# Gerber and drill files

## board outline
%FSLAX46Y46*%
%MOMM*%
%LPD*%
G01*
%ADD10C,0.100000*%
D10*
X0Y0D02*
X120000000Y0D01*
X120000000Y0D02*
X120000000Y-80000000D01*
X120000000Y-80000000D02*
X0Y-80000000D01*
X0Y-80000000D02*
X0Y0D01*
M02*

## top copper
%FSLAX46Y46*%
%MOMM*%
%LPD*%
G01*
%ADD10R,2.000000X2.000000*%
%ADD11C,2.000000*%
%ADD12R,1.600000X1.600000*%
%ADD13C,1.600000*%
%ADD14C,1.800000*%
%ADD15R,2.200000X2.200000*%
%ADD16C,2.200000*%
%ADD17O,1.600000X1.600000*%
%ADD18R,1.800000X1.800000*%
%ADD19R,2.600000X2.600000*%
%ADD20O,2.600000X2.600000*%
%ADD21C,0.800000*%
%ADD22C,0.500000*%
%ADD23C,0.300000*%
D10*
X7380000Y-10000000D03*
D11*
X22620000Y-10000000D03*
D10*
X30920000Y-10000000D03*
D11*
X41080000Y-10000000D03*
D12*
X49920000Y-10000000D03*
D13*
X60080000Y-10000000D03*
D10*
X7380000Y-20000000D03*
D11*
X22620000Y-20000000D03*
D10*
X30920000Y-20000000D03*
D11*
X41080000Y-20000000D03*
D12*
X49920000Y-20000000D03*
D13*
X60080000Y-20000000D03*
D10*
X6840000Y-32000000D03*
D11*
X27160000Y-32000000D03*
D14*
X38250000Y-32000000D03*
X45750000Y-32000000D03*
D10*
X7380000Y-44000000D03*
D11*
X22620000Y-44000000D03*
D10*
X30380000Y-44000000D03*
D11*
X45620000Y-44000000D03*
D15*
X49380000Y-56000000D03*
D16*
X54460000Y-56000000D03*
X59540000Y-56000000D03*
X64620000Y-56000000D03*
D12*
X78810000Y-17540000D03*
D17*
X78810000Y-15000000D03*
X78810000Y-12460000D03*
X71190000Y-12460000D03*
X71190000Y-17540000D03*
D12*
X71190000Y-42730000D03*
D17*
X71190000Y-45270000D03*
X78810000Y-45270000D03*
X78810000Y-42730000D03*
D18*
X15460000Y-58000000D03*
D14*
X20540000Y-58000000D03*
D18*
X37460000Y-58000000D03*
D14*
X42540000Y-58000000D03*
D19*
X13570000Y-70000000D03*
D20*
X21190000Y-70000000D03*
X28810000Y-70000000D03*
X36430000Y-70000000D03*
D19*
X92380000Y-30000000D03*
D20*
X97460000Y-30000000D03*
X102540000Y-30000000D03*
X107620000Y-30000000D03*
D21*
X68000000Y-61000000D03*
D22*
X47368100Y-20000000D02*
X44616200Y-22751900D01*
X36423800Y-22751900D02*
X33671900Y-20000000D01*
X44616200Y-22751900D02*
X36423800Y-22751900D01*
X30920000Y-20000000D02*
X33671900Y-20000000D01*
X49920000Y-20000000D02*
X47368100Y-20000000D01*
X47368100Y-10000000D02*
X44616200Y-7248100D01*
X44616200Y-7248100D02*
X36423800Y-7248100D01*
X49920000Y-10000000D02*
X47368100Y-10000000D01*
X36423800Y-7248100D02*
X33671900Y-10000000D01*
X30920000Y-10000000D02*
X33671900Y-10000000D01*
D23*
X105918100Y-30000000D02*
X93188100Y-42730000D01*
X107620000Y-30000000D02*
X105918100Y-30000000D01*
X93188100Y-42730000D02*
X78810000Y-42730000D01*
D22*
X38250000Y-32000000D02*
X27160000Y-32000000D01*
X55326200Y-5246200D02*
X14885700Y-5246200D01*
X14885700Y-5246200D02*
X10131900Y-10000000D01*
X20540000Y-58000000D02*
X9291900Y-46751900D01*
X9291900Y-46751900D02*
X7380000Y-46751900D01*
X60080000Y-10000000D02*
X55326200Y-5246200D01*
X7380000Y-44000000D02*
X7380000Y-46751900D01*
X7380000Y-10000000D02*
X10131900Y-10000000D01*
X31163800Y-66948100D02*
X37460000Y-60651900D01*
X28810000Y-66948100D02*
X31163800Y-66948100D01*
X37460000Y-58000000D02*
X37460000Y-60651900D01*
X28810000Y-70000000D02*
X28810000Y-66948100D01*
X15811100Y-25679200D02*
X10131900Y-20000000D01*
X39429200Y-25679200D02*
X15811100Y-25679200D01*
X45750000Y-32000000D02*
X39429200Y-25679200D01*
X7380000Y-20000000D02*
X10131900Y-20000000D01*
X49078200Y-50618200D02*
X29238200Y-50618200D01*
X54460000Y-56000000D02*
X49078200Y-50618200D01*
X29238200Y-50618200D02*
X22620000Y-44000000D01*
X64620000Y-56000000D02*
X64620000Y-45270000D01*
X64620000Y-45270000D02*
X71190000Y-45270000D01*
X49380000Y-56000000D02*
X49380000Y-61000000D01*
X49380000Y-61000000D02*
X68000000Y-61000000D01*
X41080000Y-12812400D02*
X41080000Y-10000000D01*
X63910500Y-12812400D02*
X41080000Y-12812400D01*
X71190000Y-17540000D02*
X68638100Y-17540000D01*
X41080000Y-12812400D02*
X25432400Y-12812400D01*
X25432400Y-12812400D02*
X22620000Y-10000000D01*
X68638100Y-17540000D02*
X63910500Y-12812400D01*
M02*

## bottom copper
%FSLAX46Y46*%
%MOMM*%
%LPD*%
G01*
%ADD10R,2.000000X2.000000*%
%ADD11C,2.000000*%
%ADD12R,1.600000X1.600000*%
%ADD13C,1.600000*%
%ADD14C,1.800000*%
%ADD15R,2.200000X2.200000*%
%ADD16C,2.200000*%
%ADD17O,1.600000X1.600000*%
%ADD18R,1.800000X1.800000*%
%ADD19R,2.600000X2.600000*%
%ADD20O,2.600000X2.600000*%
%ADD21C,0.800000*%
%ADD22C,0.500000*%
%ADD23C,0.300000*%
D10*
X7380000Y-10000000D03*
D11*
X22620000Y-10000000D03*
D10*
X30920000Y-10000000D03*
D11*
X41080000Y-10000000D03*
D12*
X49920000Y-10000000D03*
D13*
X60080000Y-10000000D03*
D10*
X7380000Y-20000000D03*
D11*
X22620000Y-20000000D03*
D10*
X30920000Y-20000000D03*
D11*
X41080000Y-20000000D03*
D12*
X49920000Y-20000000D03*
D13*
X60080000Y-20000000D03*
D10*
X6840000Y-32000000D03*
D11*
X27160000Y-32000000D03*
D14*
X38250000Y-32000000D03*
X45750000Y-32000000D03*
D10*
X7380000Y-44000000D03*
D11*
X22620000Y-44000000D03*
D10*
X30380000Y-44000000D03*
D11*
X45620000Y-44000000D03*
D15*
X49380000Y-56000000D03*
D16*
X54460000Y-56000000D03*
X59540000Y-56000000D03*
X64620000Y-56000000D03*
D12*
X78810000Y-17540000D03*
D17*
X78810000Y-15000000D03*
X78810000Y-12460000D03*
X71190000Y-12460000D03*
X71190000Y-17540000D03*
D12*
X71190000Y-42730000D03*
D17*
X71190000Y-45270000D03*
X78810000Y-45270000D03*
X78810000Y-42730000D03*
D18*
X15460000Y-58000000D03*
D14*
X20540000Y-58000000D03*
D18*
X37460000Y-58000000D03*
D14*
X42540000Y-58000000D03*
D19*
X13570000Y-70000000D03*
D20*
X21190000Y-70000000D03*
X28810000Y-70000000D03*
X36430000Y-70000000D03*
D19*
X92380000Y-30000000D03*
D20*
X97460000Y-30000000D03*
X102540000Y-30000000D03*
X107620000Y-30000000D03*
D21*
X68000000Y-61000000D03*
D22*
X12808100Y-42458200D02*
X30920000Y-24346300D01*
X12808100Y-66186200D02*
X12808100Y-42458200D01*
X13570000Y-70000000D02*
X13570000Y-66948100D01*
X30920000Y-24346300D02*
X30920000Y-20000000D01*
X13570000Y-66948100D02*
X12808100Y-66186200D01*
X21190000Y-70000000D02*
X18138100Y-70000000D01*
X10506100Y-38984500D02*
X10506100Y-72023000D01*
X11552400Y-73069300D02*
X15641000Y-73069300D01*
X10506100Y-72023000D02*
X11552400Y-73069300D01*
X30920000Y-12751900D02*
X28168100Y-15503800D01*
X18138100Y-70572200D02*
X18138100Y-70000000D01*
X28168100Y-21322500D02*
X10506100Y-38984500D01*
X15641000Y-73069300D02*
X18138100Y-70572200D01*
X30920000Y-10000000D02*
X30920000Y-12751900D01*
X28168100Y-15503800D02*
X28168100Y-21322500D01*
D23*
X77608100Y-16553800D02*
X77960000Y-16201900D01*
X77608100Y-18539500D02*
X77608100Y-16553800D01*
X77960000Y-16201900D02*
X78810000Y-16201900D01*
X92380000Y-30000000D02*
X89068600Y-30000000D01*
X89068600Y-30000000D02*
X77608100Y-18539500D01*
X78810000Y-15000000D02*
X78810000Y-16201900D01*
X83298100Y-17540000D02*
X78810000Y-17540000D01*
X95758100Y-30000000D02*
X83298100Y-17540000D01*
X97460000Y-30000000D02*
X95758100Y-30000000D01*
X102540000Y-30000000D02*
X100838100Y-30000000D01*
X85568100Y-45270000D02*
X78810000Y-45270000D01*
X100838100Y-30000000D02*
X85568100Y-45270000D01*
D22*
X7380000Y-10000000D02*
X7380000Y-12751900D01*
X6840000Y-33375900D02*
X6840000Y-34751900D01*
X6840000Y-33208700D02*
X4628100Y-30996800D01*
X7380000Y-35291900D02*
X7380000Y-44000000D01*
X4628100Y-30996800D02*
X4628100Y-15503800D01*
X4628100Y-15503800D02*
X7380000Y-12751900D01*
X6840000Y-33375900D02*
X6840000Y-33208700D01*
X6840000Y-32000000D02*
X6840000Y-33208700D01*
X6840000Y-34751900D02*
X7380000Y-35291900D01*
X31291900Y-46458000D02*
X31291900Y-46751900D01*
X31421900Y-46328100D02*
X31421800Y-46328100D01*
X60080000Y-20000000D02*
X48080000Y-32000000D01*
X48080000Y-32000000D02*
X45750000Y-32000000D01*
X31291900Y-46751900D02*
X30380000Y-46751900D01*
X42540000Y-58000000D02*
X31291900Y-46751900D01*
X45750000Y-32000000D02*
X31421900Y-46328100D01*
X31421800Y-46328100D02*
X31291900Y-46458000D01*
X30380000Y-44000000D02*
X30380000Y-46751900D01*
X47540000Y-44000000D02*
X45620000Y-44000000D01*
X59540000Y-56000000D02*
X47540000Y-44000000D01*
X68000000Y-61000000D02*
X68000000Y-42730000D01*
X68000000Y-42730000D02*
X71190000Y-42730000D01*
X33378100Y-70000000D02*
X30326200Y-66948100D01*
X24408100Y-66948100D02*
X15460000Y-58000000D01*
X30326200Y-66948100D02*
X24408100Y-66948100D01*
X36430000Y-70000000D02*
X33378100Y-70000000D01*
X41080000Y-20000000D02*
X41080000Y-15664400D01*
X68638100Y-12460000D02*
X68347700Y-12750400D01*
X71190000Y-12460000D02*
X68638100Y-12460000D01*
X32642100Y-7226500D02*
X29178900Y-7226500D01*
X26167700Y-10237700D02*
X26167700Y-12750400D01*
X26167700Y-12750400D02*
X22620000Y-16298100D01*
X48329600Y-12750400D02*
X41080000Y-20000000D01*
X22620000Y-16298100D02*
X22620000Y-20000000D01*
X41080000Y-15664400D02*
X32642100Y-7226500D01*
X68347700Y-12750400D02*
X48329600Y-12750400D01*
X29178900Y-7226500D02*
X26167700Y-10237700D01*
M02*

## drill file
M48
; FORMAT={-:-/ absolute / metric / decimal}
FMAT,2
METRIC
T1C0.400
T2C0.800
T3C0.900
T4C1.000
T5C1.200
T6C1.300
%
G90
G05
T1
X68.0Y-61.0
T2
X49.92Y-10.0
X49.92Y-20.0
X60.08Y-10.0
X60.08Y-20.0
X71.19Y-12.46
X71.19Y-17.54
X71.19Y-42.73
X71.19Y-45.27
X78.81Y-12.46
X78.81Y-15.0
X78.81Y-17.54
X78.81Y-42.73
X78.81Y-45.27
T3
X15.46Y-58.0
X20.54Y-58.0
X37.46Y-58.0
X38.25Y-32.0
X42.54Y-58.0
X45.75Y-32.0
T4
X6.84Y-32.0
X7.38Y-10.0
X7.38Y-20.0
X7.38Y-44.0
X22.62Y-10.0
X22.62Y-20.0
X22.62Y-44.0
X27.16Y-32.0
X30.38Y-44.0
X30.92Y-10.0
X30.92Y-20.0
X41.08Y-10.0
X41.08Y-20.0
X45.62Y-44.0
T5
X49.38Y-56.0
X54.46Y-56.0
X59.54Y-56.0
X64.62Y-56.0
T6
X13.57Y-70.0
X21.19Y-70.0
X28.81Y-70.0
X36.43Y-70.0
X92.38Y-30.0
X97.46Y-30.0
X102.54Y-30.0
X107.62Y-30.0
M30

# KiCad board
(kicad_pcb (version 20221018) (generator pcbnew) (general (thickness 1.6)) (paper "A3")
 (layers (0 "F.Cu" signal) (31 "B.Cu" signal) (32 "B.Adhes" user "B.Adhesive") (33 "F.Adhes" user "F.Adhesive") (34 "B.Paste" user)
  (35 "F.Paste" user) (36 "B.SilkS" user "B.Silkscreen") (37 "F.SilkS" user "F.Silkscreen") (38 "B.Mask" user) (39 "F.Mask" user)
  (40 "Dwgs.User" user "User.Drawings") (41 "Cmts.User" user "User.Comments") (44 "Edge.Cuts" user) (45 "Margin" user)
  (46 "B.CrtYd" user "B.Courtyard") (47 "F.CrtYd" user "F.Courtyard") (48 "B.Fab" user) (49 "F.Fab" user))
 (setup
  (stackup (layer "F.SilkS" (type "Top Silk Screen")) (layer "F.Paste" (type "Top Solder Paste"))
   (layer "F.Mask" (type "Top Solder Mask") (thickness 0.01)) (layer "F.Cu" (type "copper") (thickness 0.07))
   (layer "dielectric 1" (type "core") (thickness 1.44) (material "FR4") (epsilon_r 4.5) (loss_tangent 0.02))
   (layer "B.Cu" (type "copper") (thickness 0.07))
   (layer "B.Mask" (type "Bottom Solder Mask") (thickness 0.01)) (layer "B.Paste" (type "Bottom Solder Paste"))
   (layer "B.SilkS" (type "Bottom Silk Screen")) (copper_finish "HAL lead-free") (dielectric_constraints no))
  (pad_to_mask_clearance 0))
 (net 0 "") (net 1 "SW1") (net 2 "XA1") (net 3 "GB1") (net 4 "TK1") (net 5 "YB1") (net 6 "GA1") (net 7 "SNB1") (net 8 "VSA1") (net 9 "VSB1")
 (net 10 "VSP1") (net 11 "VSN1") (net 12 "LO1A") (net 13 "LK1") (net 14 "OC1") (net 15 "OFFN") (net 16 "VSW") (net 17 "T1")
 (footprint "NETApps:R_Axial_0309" (layer "F.Cu") (at 15 10)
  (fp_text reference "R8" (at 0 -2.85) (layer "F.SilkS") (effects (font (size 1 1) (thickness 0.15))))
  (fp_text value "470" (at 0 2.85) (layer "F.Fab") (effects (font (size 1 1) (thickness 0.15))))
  (pad "1" thru_hole rect (at -7.62 0) (size 2 2) (drill 1) (layers "*.Cu" "*.Mask") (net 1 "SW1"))
  (pad "2" thru_hole circle (at 7.62 0) (size 2 2) (drill 1) (layers "*.Cu" "*.Mask") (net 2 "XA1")))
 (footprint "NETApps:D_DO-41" (layer "F.Cu") (at 36 10)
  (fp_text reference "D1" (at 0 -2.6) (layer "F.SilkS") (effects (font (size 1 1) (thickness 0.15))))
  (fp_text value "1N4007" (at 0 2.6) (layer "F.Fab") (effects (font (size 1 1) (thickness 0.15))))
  (pad "1" thru_hole rect (at -5.08 0) (size 2 2) (drill 1) (layers "*.Cu" "*.Mask") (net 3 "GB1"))
  (pad "2" thru_hole circle (at 5.08 0) (size 2 2) (drill 1) (layers "*.Cu" "*.Mask") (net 2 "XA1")))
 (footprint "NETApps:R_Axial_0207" (layer "F.Cu") (at 55 10)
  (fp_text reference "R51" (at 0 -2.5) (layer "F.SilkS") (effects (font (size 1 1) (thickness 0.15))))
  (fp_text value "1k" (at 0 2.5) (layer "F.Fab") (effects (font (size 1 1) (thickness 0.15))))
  (pad "1" thru_hole rect (at -5.08 0) (size 1.6 1.6) (drill 0.8) (layers "*.Cu" "*.Mask") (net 3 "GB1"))
  (pad "2" thru_hole circle (at 5.08 0) (size 1.6 1.6) (drill 0.8) (layers "*.Cu" "*.Mask") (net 1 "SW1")))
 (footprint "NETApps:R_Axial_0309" (layer "F.Cu") (at 15 20)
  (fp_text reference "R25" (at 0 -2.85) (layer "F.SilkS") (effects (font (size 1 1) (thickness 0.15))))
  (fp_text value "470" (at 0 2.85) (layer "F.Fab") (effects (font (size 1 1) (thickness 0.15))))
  (pad "1" thru_hole rect (at -7.62 0) (size 2 2) (drill 1) (layers "*.Cu" "*.Mask") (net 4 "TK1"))
  (pad "2" thru_hole circle (at 7.62 0) (size 2 2) (drill 1) (layers "*.Cu" "*.Mask") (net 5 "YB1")))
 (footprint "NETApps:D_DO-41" (layer "F.Cu") (at 36 20)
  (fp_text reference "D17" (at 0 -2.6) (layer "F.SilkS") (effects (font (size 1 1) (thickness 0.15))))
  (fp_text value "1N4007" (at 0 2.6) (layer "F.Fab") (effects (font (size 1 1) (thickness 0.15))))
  (pad "1" thru_hole rect (at -5.08 0) (size 2 2) (drill 1) (layers "*.Cu" "*.Mask") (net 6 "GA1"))
  (pad "2" thru_hole circle (at 5.08 0) (size 2 2) (drill 1) (layers "*.Cu" "*.Mask") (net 5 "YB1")))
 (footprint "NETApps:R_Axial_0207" (layer "F.Cu") (at 55 20)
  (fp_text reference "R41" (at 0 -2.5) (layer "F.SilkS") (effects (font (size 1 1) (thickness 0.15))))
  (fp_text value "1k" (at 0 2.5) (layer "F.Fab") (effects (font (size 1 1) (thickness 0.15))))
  (pad "1" thru_hole rect (at -5.08 0) (size 1.6 1.6) (drill 0.8) (layers "*.Cu" "*.Mask") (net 6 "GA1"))
  (pad "2" thru_hole circle (at 5.08 0) (size 1.6 1.6) (drill 0.8) (layers "*.Cu" "*.Mask") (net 4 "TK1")))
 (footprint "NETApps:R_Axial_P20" (layer "F.Cu") (at 17 32)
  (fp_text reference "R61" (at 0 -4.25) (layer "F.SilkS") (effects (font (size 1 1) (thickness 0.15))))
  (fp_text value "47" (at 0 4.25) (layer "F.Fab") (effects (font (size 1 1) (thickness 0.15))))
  (pad "1" thru_hole rect (at -10.16 0) (size 2 2) (drill 1) (layers "*.Cu" "*.Mask") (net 1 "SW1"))
  (pad "2" thru_hole circle (at 10.16 0) (size 2 2) (drill 1) (layers "*.Cu" "*.Mask") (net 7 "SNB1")))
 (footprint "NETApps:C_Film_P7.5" (layer "F.Cu") (at 42 32)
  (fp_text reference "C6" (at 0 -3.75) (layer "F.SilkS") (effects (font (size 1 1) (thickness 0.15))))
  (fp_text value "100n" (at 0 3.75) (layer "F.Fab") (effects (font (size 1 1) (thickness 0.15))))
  (pad "1" thru_hole circle (at -3.75 0) (size 1.8 1.8) (drill 0.9) (layers "*.Cu" "*.Mask") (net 7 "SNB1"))
  (pad "2" thru_hole circle (at 3.75 0) (size 1.8 1.8) (drill 0.9) (layers "*.Cu" "*.Mask") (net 4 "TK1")))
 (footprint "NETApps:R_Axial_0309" (layer "F.Cu") (at 15 44)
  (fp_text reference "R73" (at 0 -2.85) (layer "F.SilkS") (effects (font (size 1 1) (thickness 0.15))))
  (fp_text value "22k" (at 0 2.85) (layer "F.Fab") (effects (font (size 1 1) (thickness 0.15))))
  (pad "1" thru_hole rect (at -7.62 0) (size 2 2) (drill 1) (layers "*.Cu" "*.Mask") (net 1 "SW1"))
  (pad "2" thru_hole circle (at 7.62 0) (size 2 2) (drill 1) (layers "*.Cu" "*.Mask") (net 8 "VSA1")))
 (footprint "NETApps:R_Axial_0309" (layer "F.Cu") (at 38 44)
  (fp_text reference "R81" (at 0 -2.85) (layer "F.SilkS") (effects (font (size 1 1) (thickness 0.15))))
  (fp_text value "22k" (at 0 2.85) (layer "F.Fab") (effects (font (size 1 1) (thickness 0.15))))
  (pad "1" thru_hole rect (at -7.62 0) (size 2 2) (drill 1) (layers "*.Cu" "*.Mask") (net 4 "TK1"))
  (pad "2" thru_hole circle (at 7.62 0) (size 2 2) (drill 1) (layers "*.Cu" "*.Mask") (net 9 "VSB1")))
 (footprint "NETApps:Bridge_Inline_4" (layer "F.Cu") (at 57 56)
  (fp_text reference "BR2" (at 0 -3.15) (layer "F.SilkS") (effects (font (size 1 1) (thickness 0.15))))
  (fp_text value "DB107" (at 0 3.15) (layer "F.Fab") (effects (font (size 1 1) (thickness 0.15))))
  (pad "1" thru_hole rect (at -7.62 0) (size 2.2 2.2) (drill 1.2) (layers "*.Cu" "*.Mask") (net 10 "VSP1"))
  (pad "2" thru_hole circle (at -2.54 0) (size 2.2 2.2) (drill 1.2) (layers "*.Cu" "*.Mask") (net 8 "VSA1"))
  (pad "3" thru_hole circle (at 2.54 0) (size 2.2 2.2) (drill 1.2) (layers "*.Cu" "*.Mask") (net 9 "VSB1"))
  (pad "4" thru_hole circle (at 7.62 0) (size 2.2 2.2) (drill 1.2) (layers "*.Cu" "*.Mask") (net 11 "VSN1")))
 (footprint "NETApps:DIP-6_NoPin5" (layer "F.Cu") (at 75 15 180)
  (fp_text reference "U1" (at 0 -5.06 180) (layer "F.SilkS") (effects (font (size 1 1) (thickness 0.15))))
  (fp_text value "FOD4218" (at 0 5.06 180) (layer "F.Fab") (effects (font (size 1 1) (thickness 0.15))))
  (pad "1" thru_hole rect (at -3.81 -2.54) (size 1.6 1.6) (drill 0.8) (layers "*.Cu" "*.Mask") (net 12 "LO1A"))
  (pad "2" thru_hole oval (at -3.81 0) (size 1.6 1.6) (drill 0.8) (layers "*.Cu" "*.Mask") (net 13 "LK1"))
  (pad "3" thru_hole oval (at -3.81 2.54) (size 1.6 1.6) (drill 0.8) (layers "*.Cu" "*.Mask"))
  (pad "4" thru_hole oval (at 3.81 2.54) (size 1.6 1.6) (drill 0.8) (layers "*.Cu" "*.Mask") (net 5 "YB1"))
  (pad "6" thru_hole oval (at 3.81 -2.54) (size 1.6 1.6) (drill 0.8) (layers "*.Cu" "*.Mask") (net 2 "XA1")))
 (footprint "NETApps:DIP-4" (layer "F.Cu") (at 75 44)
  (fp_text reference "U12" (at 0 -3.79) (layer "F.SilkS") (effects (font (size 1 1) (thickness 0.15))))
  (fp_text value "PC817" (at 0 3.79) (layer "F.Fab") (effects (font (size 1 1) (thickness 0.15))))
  (pad "1" thru_hole rect (at -3.81 -1.27) (size 1.6 1.6) (drill 0.8) (layers "*.Cu" "*.Mask") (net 10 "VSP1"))
  (pad "2" thru_hole oval (at -3.81 1.27) (size 1.6 1.6) (drill 0.8) (layers "*.Cu" "*.Mask") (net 11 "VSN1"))
  (pad "3" thru_hole oval (at 3.81 1.27) (size 1.6 1.6) (drill 0.8) (layers "*.Cu" "*.Mask") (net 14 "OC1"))
  (pad "4" thru_hole oval (at 3.81 -1.27) (size 1.6 1.6) (drill 0.8) (layers "*.Cu" "*.Mask") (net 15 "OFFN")))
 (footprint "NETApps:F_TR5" (layer "F.Cu") (at 18 58)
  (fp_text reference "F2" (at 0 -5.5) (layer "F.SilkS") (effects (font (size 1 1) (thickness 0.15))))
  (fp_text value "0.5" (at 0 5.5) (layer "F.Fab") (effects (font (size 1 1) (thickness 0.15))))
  (pad "1" thru_hole rect (at -2.54 0) (size 1.8 1.8) (drill 0.9) (layers "*.Cu" "*.Mask") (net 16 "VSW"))
  (pad "2" thru_hole circle (at 2.54 0) (size 1.8 1.8) (drill 0.9) (layers "*.Cu" "*.Mask") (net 1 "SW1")))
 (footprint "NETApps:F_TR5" (layer "F.Cu") (at 40 58)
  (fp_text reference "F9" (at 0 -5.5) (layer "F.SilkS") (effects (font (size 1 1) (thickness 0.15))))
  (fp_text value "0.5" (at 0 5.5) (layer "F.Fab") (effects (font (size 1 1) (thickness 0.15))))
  (pad "1" thru_hole rect (at -2.54 0) (size 1.8 1.8) (drill 0.9) (layers "*.Cu" "*.Mask") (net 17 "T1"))
  (pad "2" thru_hole circle (at 2.54 0) (size 1.8 1.8) (drill 0.9) (layers "*.Cu" "*.Mask") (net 4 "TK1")))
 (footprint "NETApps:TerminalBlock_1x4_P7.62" (layer "F.Cu") (at 25 70)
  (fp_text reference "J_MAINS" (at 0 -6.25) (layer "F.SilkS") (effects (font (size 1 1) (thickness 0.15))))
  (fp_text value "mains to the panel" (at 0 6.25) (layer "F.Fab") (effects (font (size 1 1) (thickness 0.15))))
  (pad "1" thru_hole rect (at -11.43 0) (size 2.6 2.6) (drill 1.3) (layers "*.Cu" "*.Mask") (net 6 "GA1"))
  (pad "2" thru_hole oval (at -3.81 0) (size 2.6 2.6) (drill 1.3) (layers "*.Cu" "*.Mask") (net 3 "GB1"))
  (pad "3" thru_hole oval (at 3.81 0) (size 2.6 2.6) (drill 1.3) (layers "*.Cu" "*.Mask") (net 17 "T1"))
  (pad "4" thru_hole oval (at 11.43 0) (size 2.6 2.6) (drill 1.3) (layers "*.Cu" "*.Mask") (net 16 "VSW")))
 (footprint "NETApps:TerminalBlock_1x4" (layer "F.Cu") (at 100 30)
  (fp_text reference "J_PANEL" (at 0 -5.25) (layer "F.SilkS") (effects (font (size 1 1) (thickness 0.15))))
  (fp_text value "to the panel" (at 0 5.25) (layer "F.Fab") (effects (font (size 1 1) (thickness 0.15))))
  (pad "1" thru_hole rect (at -7.62 0) (size 2.6 2.6) (drill 1.3) (layers "*.Cu" "*.Mask") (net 13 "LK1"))
  (pad "2" thru_hole oval (at -2.54 0) (size 2.6 2.6) (drill 1.3) (layers "*.Cu" "*.Mask") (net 12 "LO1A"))
  (pad "3" thru_hole oval (at 2.54 0) (size 2.6 2.6) (drill 1.3) (layers "*.Cu" "*.Mask") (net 14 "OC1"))
  (pad "4" thru_hole oval (at 7.62 0) (size 2.6 2.6) (drill 1.3) (layers "*.Cu" "*.Mask") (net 15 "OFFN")))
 (gr_line (start 0 0) (end 120 0) (stroke (width 0.1) (type solid)) (layer "Edge.Cuts"))
 (gr_line (start 120 0) (end 120 80) (stroke (width 0.1) (type solid)) (layer "Edge.Cuts"))
 (gr_line (start 120 80) (end 0 80) (stroke (width 0.1) (type solid)) (layer "Edge.Cuts"))
 (gr_line (start 0 80) (end 0 0) (stroke (width 0.1) (type solid)) (layer "Edge.Cuts"))
 (segment locked (start 47.3681 20) (end 44.6162 22.7519) (width 0.5) (layer "F.Cu") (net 6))
 (segment locked (start 36.4238 22.7519) (end 33.6719 20) (width 0.5) (layer "F.Cu") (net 6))
 (segment locked (start 44.6162 22.7519) (end 36.4238 22.7519) (width 0.5) (layer "F.Cu") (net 6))
 (segment locked (start 30.92 20) (end 33.6719 20) (width 0.5) (layer "F.Cu") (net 6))
 (segment locked (start 49.92 20) (end 47.3681 20) (width 0.5) (layer "F.Cu") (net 6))
 (segment locked (start 12.8081 42.4582) (end 30.92 24.3463) (width 0.5) (layer "B.Cu") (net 6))
 (segment locked (start 12.8081 66.1862) (end 12.8081 42.4582) (width 0.5) (layer "B.Cu") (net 6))
 (segment locked (start 13.57 70) (end 13.57 66.9481) (width 0.5) (layer "B.Cu") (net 6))
 (segment locked (start 30.92 24.3463) (end 30.92 20) (width 0.5) (layer "B.Cu") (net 6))
 (segment locked (start 13.57 66.9481) (end 12.8081 66.1862) (width 0.5) (layer "B.Cu") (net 6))
 (segment locked (start 47.3681 10) (end 44.6162 7.2481) (width 0.5) (layer "F.Cu") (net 3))
 (segment locked (start 44.6162 7.2481) (end 36.4238 7.2481) (width 0.5) (layer "F.Cu") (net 3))
 (segment locked (start 49.92 10) (end 47.3681 10) (width 0.5) (layer "F.Cu") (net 3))
 (segment locked (start 36.4238 7.2481) (end 33.6719 10) (width 0.5) (layer "F.Cu") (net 3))
 (segment locked (start 30.92 10) (end 33.6719 10) (width 0.5) (layer "F.Cu") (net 3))
 (segment locked (start 21.19 70) (end 18.1381 70) (width 0.5) (layer "B.Cu") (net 3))
 (segment locked (start 10.5061 38.9845) (end 10.5061 72.023) (width 0.5) (layer "B.Cu") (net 3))
 (segment locked (start 11.5524 73.0693) (end 15.641 73.0693) (width 0.5) (layer "B.Cu") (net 3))
 (segment locked (start 10.5061 72.023) (end 11.5524 73.0693) (width 0.5) (layer "B.Cu") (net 3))
 (segment locked (start 30.92 12.7519) (end 28.1681 15.5038) (width 0.5) (layer "B.Cu") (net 3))
 (segment locked (start 18.1381 70.5722) (end 18.1381 70) (width 0.5) (layer "B.Cu") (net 3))
 (segment locked (start 28.1681 21.3225) (end 10.5061 38.9845) (width 0.5) (layer "B.Cu") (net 3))
 (segment locked (start 15.641 73.0693) (end 18.1381 70.5722) (width 0.5) (layer "B.Cu") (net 3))
 (segment locked (start 30.92 10) (end 30.92 12.7519) (width 0.5) (layer "B.Cu") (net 3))
 (segment locked (start 28.1681 15.5038) (end 28.1681 21.3225) (width 0.5) (layer "B.Cu") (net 3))
 (segment (start 77.6081 16.5538) (end 77.96 16.2019) (width 0.3) (layer "B.Cu") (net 13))
 (segment (start 77.6081 18.5395) (end 77.6081 16.5538) (width 0.3) (layer "B.Cu") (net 13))
 (segment (start 77.96 16.2019) (end 78.81 16.2019) (width 0.3) (layer "B.Cu") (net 13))
 (segment (start 92.38 30) (end 89.0686 30) (width 0.3) (layer "B.Cu") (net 13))
 (segment (start 89.0686 30) (end 77.6081 18.5395) (width 0.3) (layer "B.Cu") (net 13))
 (segment (start 78.81 15) (end 78.81 16.2019) (width 0.3) (layer "B.Cu") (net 13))
 (segment (start 83.2981 17.54) (end 78.81 17.54) (width 0.3) (layer "B.Cu") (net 12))
 (segment (start 95.7581 30) (end 83.2981 17.54) (width 0.3) (layer "B.Cu") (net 12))
 (segment (start 97.46 30) (end 95.7581 30) (width 0.3) (layer "B.Cu") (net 12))
 (segment (start 102.54 30) (end 100.8381 30) (width 0.3) (layer "B.Cu") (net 14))
 (segment (start 85.5681 45.27) (end 78.81 45.27) (width 0.3) (layer "B.Cu") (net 14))
 (segment (start 100.8381 30) (end 85.5681 45.27) (width 0.3) (layer "B.Cu") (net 14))
 (segment (start 105.9181 30) (end 93.1881 42.73) (width 0.3) (layer "F.Cu") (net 15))
 (segment (start 107.62 30) (end 105.9181 30) (width 0.3) (layer "F.Cu") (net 15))
 (segment (start 93.1881 42.73) (end 78.81 42.73) (width 0.3) (layer "F.Cu") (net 15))
 (segment locked (start 38.25 32) (end 27.16 32) (width 0.5) (layer "F.Cu") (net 7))
 (segment locked (start 55.3262 5.2462) (end 14.8857 5.2462) (width 0.5) (layer "F.Cu") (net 1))
 (segment locked (start 14.8857 5.2462) (end 10.1319 10) (width 0.5) (layer "F.Cu") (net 1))
 (segment locked (start 20.54 58) (end 9.2919 46.7519) (width 0.5) (layer "F.Cu") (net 1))
 (segment locked (start 9.2919 46.7519) (end 7.38 46.7519) (width 0.5) (layer "F.Cu") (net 1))
 (segment locked (start 60.08 10) (end 55.3262 5.2462) (width 0.5) (layer "F.Cu") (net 1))
 (segment locked (start 7.38 44) (end 7.38 46.7519) (width 0.5) (layer "F.Cu") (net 1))
 (segment locked (start 7.38 10) (end 10.1319 10) (width 0.5) (layer "F.Cu") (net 1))
 (segment locked (start 7.38 10) (end 7.38 12.7519) (width 0.5) (layer "B.Cu") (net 1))
 (segment locked (start 6.84 33.3759) (end 6.84 34.7519) (width 0.5) (layer "B.Cu") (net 1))
 (segment locked (start 6.84 33.2087) (end 4.6281 30.9968) (width 0.5) (layer "B.Cu") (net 1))
 (segment locked (start 7.38 35.2919) (end 7.38 44) (width 0.5) (layer "B.Cu") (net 1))
 (segment locked (start 4.6281 30.9968) (end 4.6281 15.5038) (width 0.5) (layer "B.Cu") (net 1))
 (segment locked (start 4.6281 15.5038) (end 7.38 12.7519) (width 0.5) (layer "B.Cu") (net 1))
 (segment locked (start 6.84 33.3759) (end 6.84 33.2087) (width 0.5) (layer "B.Cu") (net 1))
 (segment locked (start 6.84 32) (end 6.84 33.2087) (width 0.5) (layer "B.Cu") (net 1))
 (segment locked (start 6.84 34.7519) (end 7.38 35.2919) (width 0.5) (layer "B.Cu") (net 1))
 (segment locked (start 31.1638 66.9481) (end 37.46 60.6519) (width 0.5) (layer "F.Cu") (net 17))
 (segment locked (start 28.81 66.9481) (end 31.1638 66.9481) (width 0.5) (layer "F.Cu") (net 17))
 (segment locked (start 37.46 58) (end 37.46 60.6519) (width 0.5) (layer "F.Cu") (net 17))
 (segment locked (start 28.81 70) (end 28.81 66.9481) (width 0.5) (layer "F.Cu") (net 17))
 (segment locked (start 15.8111 25.6792) (end 10.1319 20) (width 0.5) (layer "F.Cu") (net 4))
 (segment locked (start 39.4292 25.6792) (end 15.8111 25.6792) (width 0.5) (layer "F.Cu") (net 4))
 (segment locked (start 45.75 32) (end 39.4292 25.6792) (width 0.5) (layer "F.Cu") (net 4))
 (segment locked (start 7.38 20) (end 10.1319 20) (width 0.5) (layer "F.Cu") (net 4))
 (segment locked (start 31.2919 46.458) (end 31.2919 46.7519) (width 0.5) (layer "B.Cu") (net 4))
 (segment locked (start 31.4219 46.3281) (end 31.4218 46.3281) (width 0.5) (layer "B.Cu") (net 4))
 (segment locked (start 60.08 20) (end 48.08 32) (width 0.5) (layer "B.Cu") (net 4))
 (segment locked (start 48.08 32) (end 45.75 32) (width 0.5) (layer "B.Cu") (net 4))
 (segment locked (start 31.2919 46.7519) (end 30.38 46.7519) (width 0.5) (layer "B.Cu") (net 4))
 (segment locked (start 42.54 58) (end 31.2919 46.7519) (width 0.5) (layer "B.Cu") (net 4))
 (segment locked (start 45.75 32) (end 31.4219 46.3281) (width 0.5) (layer "B.Cu") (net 4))
 (segment locked (start 31.4218 46.3281) (end 31.2919 46.458) (width 0.5) (layer "B.Cu") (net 4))
 (segment locked (start 30.38 44) (end 30.38 46.7519) (width 0.5) (layer "B.Cu") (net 4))
 (segment locked (start 49.0782 50.6182) (end 29.2382 50.6182) (width 0.5) (layer "F.Cu") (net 8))
 (segment locked (start 54.46 56) (end 49.0782 50.6182) (width 0.5) (layer "F.Cu") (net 8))
 (segment locked (start 29.2382 50.6182) (end 22.62 44) (width 0.5) (layer "F.Cu") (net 8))
 (segment locked (start 47.54 44) (end 45.62 44) (width 0.5) (layer "B.Cu") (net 9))
 (segment locked (start 59.54 56) (end 47.54 44) (width 0.5) (layer "B.Cu") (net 9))
 (segment locked (start 64.62 56) (end 64.62 45.27) (width 0.5) (layer "F.Cu") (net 11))
 (segment locked (start 64.62 45.27) (end 71.19 45.27) (width 0.5) (layer "F.Cu") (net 11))
 (segment locked (start 49.38 56) (end 49.38 61) (width 0.5) (layer "F.Cu") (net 10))
 (segment locked (start 49.38 61) (end 68 61) (width 0.5) (layer "F.Cu") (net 10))
 (via locked (at 68 61) (size 0.8) (drill 0.4) (layers "F.Cu" "B.Cu") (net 10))
 (segment locked (start 68 61) (end 68 42.73) (width 0.5) (layer "B.Cu") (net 10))
 (segment locked (start 68 42.73) (end 71.19 42.73) (width 0.5) (layer "B.Cu") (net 10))
 (segment locked (start 33.3781 70) (end 30.3262 66.9481) (width 0.5) (layer "B.Cu") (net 16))
 (segment locked (start 24.4081 66.9481) (end 15.46 58) (width 0.5) (layer "B.Cu") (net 16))
 (segment locked (start 30.3262 66.9481) (end 24.4081 66.9481) (width 0.5) (layer "B.Cu") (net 16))
 (segment locked (start 36.43 70) (end 33.3781 70) (width 0.5) (layer "B.Cu") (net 16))
 (segment locked (start 41.08 12.8124) (end 41.08 10) (width 0.5) (layer "F.Cu") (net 2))
 (segment locked (start 63.9105 12.8124) (end 41.08 12.8124) (width 0.5) (layer "F.Cu") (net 2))
 (segment locked (start 71.19 17.54) (end 68.6381 17.54) (width 0.5) (layer "F.Cu") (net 2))
 (segment locked (start 41.08 12.8124) (end 25.4324 12.8124) (width 0.5) (layer "F.Cu") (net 2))
 (segment locked (start 25.4324 12.8124) (end 22.62 10) (width 0.5) (layer "F.Cu") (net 2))
 (segment locked (start 68.6381 17.54) (end 63.9105 12.8124) (width 0.5) (layer "F.Cu") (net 2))
 (segment locked (start 41.08 20) (end 41.08 15.6644) (width 0.5) (layer "B.Cu") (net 5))
 (segment locked (start 68.6381 12.46) (end 68.3477 12.7504) (width 0.5) (layer "B.Cu") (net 5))
 (segment locked (start 71.19 12.46) (end 68.6381 12.46) (width 0.5) (layer "B.Cu") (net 5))
 (segment locked (start 32.6421 7.2265) (end 29.1789 7.2265) (width 0.5) (layer "B.Cu") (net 5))
 (segment locked (start 26.1677 10.2377) (end 26.1677 12.7504) (width 0.5) (layer "B.Cu") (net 5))
 (segment locked (start 26.1677 12.7504) (end 22.62 16.2981) (width 0.5) (layer "B.Cu") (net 5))
 (segment locked (start 48.3296 12.7504) (end 41.08 20) (width 0.5) (layer "B.Cu") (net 5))
 (segment locked (start 22.62 16.2981) (end 22.62 20) (width 0.5) (layer "B.Cu") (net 5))
 (segment locked (start 41.08 15.6644) (end 32.6421 7.2265) (width 0.5) (layer "B.Cu") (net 5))
 (segment locked (start 68.3477 12.7504) (end 48.3296 12.7504) (width 0.5) (layer "B.Cu") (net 5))
 (segment locked (start 29.1789 7.2265) (end 26.1677 10.2377) (width 0.5) (layer "B.Cu") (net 5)))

